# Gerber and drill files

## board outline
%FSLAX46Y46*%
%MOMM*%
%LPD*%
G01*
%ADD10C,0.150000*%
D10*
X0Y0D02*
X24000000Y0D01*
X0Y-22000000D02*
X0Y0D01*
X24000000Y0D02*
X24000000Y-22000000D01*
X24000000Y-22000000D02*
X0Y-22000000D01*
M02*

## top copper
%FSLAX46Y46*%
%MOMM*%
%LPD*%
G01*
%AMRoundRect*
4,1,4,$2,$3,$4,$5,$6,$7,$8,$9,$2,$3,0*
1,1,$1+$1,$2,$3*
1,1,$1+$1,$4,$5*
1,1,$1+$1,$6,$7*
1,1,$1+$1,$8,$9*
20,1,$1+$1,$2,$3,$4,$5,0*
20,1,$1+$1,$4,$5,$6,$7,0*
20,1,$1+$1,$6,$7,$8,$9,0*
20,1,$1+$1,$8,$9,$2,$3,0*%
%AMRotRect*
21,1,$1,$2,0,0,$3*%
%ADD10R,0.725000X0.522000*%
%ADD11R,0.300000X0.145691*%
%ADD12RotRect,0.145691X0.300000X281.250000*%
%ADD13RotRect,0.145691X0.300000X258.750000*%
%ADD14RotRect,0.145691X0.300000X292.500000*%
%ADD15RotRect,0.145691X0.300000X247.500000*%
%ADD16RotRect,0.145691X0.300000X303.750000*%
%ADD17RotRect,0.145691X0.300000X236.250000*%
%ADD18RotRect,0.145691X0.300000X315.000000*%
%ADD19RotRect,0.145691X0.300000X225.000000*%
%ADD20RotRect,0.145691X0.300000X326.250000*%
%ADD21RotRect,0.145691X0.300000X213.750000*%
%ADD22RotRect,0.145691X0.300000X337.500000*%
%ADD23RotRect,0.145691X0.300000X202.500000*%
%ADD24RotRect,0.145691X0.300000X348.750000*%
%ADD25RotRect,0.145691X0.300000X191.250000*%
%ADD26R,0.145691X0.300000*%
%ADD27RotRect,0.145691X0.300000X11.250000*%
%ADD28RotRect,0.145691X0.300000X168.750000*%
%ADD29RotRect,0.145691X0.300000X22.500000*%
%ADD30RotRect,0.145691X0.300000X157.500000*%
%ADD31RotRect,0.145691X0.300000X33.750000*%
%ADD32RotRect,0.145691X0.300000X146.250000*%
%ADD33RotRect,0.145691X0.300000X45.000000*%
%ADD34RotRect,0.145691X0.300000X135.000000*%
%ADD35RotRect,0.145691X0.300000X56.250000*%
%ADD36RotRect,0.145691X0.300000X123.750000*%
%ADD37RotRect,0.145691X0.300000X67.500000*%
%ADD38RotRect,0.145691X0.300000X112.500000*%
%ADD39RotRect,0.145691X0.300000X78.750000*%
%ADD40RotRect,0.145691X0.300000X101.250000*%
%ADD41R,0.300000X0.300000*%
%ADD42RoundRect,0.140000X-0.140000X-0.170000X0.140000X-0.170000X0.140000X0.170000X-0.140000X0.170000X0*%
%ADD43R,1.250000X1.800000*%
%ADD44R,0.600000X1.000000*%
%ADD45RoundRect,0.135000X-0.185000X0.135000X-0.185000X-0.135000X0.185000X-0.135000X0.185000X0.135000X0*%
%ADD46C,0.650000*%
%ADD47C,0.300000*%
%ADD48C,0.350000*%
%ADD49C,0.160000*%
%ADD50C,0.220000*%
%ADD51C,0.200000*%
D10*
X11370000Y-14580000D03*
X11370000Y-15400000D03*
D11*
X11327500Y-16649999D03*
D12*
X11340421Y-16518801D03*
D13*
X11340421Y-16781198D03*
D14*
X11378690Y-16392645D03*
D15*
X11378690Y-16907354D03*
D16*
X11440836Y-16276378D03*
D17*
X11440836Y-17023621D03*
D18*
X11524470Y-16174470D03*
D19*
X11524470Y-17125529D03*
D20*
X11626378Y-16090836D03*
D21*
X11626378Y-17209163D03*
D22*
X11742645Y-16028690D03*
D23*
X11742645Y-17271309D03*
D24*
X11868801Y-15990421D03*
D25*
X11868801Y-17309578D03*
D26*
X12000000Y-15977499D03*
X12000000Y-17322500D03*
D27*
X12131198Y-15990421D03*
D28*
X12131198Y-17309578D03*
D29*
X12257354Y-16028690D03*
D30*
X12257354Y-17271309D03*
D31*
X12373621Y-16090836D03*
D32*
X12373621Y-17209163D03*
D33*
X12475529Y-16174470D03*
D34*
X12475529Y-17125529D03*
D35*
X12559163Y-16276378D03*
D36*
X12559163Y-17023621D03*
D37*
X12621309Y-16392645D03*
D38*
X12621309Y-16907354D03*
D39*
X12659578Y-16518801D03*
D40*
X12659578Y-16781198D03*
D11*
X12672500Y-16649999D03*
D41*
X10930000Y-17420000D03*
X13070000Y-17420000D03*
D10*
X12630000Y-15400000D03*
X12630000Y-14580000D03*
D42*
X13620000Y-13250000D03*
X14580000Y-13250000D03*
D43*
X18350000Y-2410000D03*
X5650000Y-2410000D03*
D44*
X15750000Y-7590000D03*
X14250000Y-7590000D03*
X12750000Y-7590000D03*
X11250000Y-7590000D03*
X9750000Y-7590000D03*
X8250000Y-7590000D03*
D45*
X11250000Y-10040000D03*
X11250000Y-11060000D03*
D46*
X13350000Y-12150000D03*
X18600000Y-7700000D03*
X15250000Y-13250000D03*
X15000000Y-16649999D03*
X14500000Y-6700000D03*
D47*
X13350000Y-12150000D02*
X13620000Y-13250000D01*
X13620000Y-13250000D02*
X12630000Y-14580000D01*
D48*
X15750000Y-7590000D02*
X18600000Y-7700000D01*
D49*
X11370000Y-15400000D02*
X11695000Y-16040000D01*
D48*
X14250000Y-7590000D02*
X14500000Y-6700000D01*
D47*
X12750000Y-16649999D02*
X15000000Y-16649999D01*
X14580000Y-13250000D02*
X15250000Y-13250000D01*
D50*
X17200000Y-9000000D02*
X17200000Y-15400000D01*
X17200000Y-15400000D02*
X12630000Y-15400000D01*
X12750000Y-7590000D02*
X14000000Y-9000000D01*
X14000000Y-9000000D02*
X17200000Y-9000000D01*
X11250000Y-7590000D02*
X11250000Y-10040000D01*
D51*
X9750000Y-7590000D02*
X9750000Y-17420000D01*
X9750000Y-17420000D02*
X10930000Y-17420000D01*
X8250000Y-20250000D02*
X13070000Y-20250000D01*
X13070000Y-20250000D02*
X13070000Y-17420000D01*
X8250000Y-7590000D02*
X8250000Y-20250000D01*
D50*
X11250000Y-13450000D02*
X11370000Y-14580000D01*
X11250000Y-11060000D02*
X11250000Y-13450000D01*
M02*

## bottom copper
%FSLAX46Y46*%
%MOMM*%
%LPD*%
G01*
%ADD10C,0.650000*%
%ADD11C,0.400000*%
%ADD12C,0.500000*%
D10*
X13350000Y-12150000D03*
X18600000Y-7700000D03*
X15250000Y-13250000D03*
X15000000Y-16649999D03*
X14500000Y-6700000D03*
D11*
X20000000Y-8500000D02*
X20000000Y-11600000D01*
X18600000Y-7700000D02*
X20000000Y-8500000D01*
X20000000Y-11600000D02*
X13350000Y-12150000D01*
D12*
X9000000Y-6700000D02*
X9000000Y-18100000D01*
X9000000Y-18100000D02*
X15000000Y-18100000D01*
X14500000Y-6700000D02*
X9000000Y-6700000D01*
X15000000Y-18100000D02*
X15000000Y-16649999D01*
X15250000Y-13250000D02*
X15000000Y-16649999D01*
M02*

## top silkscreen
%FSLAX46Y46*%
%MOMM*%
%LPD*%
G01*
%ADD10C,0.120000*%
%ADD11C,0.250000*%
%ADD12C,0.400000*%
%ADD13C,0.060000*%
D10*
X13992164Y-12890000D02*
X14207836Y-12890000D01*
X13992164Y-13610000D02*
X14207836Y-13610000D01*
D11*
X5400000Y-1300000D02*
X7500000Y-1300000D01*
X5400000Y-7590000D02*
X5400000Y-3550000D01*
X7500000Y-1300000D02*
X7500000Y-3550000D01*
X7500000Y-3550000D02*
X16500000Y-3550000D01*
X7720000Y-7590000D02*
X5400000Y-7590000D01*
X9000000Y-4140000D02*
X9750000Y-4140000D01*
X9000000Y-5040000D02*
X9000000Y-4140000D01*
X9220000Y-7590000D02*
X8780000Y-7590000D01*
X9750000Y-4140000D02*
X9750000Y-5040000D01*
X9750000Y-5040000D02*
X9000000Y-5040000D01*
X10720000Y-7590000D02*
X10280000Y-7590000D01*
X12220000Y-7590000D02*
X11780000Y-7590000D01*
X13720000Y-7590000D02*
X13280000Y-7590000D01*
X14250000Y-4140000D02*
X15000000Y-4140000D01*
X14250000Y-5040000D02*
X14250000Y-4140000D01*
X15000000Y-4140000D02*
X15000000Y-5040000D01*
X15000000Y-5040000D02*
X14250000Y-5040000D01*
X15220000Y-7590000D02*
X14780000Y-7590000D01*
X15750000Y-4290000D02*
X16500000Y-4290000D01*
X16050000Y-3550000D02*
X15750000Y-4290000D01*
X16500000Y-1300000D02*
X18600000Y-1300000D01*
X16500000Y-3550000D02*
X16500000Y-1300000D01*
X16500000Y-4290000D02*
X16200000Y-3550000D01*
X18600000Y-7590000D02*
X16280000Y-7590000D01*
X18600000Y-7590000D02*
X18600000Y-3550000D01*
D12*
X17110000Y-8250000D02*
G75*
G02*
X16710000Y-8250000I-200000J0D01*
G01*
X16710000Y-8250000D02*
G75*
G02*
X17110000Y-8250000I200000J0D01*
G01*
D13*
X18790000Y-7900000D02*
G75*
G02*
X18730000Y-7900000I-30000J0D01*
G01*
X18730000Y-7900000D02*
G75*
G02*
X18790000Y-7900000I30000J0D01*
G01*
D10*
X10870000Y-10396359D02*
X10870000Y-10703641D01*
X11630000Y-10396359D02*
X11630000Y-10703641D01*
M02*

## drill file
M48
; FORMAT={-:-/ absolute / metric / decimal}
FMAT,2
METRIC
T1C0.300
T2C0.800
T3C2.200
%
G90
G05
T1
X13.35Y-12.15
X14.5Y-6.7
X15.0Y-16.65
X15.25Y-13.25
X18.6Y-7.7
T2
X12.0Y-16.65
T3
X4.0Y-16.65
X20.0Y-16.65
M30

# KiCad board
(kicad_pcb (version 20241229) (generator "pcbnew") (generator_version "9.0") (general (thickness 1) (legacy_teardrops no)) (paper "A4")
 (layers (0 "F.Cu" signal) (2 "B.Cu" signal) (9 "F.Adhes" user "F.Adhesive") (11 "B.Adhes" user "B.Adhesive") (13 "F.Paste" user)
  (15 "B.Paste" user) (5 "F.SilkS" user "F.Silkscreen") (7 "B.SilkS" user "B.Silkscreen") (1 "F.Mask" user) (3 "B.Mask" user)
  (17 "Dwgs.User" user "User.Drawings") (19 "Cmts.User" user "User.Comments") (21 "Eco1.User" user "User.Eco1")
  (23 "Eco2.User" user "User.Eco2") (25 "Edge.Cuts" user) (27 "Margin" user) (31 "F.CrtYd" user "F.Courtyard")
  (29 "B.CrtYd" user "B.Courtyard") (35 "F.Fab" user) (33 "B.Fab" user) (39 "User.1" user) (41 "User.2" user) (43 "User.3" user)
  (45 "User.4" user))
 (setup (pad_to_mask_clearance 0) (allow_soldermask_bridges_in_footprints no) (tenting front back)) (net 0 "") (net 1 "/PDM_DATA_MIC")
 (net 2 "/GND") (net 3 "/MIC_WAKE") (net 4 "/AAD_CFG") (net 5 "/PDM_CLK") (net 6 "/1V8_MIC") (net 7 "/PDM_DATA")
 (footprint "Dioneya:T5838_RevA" (layer "F.Cu") (at 12 16)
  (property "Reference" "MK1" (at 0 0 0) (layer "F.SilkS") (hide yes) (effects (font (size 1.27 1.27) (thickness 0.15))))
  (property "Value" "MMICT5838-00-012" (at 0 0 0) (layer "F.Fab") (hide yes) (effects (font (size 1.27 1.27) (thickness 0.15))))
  (pad "" np_thru_hole circle (at 0 0.649999) (size 0.8 0.8) (drill 0.8) (layers "*.Cu" "*.Mask"))
  (pad "1" smd rect (at -0.63 -1.42 90) (size 0.522 0.725) (layers "F.Cu" "F.Mask" "F.Paste") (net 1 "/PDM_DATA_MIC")
   (solder_paste_margin -0.05) (thermal_bridge_angle 45))
  (pad "2" smd rect (at -0.63 -0.6 90) (size 0.522 0.725) (layers "F.Cu" "F.Mask" "F.Paste") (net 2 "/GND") (solder_paste_margin -0.05)
   (thermal_bridge_angle 45))
  (pad "3" smd rect (at -0.6725 0.649999 270) (size 0.145691 0.3) (layers "F.Cu" "F.Mask") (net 2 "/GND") (thermal_bridge_angle 45))
  (pad "3" smd rect (at -0.659579 0.518801 281.25) (size 0.145691 0.3) (layers "F.Cu" "F.Mask") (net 2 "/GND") (thermal_bridge_angle 45))
  (pad "3" smd rect (at -0.659579 0.781198 258.75) (size 0.145691 0.3) (layers "F.Cu" "F.Mask") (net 2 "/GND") (thermal_bridge_angle 45))
  (pad "3" smd rect (at -0.62131 0.392645 292.5) (size 0.145691 0.3) (layers "F.Cu" "F.Mask") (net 2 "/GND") (thermal_bridge_angle 45))
  (pad "3" smd rect (at -0.62131 0.907354 247.5) (size 0.145691 0.3) (layers "F.Cu" "F.Mask") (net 2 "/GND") (thermal_bridge_angle 45))
  (pad "3" smd rect (at -0.559164 0.276378 303.75) (size 0.145691 0.3) (layers "F.Cu" "F.Mask") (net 2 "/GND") (thermal_bridge_angle 45))
  (pad "3" smd rect (at -0.559164 1.023621 236.25) (size 0.145691 0.3) (layers "F.Cu" "F.Mask") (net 2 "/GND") (thermal_bridge_angle 45))
  (pad "3" smd rect (at -0.47553 0.17447 315) (size 0.145691 0.3) (layers "F.Cu" "F.Mask") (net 2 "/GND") (thermal_bridge_angle 45))
  (pad "3" smd rect (at -0.47553 1.125529 225) (size 0.145691 0.3) (layers "F.Cu" "F.Mask") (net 2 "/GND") (thermal_bridge_angle 45))
  (pad "3" smd rect (at -0.373622 0.090836 326.25) (size 0.145691 0.3) (layers "F.Cu" "F.Mask") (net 2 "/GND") (thermal_bridge_angle 45))
  (pad "3" smd rect (at -0.373622 1.209163 213.75) (size 0.145691 0.3) (layers "F.Cu" "F.Mask") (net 2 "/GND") (thermal_bridge_angle 45))
  (pad "3" smd rect (at -0.257355 0.02869 337.5) (size 0.145691 0.3) (layers "F.Cu" "F.Mask") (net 2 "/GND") (thermal_bridge_angle 45))
  (pad "3" smd rect (at -0.257355 1.271309 202.5) (size 0.145691 0.3) (layers "F.Cu" "F.Mask") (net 2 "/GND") (thermal_bridge_angle 45))
  (pad "3" smd rect (at -0.131199 -0.009579 348.75) (size 0.145691 0.3) (layers "F.Cu" "F.Mask") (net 2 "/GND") (thermal_bridge_angle 45))
  (pad "3" smd rect (at -0.131199 1.309578 191.25) (size 0.145691 0.3) (layers "F.Cu" "F.Mask") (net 2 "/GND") (thermal_bridge_angle 45))
  (pad "3" smd rect (at 0 -0.022501) (size 0.145691 0.3) (layers "F.Cu" "F.Mask") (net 2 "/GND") (thermal_bridge_angle 45))
  (pad "3" smd rect (at 0 1.3225 180) (size 0.145691 0.3) (layers "F.Cu" "F.Mask") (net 2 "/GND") (thermal_bridge_angle 45))
  (pad "3" smd rect (at 0.131198 -0.009579 11.25) (size 0.145691 0.3) (layers "F.Cu" "F.Mask") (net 2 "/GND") (thermal_bridge_angle 45))
  (pad "3" smd rect (at 0.131198 1.309578 168.75) (size 0.145691 0.3) (layers "F.Cu" "F.Mask") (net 2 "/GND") (thermal_bridge_angle 45))
  (pad "3" smd rect (at 0.257354 0.02869 22.5) (size 0.145691 0.3) (layers "F.Cu" "F.Mask") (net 2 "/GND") (thermal_bridge_angle 45))
  (pad "3" smd rect (at 0.257354 1.271309 157.5) (size 0.145691 0.3) (layers "F.Cu" "F.Mask") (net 2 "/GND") (thermal_bridge_angle 45))
  (pad "3" smd rect (at 0.373621 0.090836 33.75) (size 0.145691 0.3) (layers "F.Cu" "F.Mask") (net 2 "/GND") (thermal_bridge_angle 45))
  (pad "3" smd rect (at 0.373621 1.209163 146.25) (size 0.145691 0.3) (layers "F.Cu" "F.Mask") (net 2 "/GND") (thermal_bridge_angle 45))
  (pad "3" smd rect (at 0.475529 0.17447 45) (size 0.145691 0.3) (layers "F.Cu" "F.Mask") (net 2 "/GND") (thermal_bridge_angle 45))
  (pad "3" smd rect (at 0.475529 1.125529 135) (size 0.145691 0.3) (layers "F.Cu" "F.Mask") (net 2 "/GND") (thermal_bridge_angle 45))
  (pad "3" smd rect (at 0.559163 0.276378 56.25) (size 0.145691 0.3) (layers "F.Cu" "F.Mask") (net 2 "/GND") (thermal_bridge_angle 45))
  (pad "3" smd rect (at 0.559163 1.023621 123.75) (size 0.145691 0.3) (layers "F.Cu" "F.Mask") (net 2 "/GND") (thermal_bridge_angle 45))
  (pad "3" smd rect (at 0.621309 0.392645 67.5) (size 0.145691 0.3) (layers "F.Cu" "F.Mask") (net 2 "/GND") (thermal_bridge_angle 45))
  (pad "3" smd rect (at 0.621309 0.907354 112.5) (size 0.145691 0.3) (layers "F.Cu" "F.Mask") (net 2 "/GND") (thermal_bridge_angle 45))
  (pad "3" smd rect (at 0.659578 0.518801 78.75) (size 0.145691 0.3) (layers "F.Cu" "F.Mask") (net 2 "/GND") (thermal_bridge_angle 45))
  (pad "3" smd rect (at 0.659578 0.781198 101.25) (size 0.145691 0.3) (layers "F.Cu" "F.Mask") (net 2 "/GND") (thermal_bridge_angle 45))
  (pad "3" smd rect (at 0.6725 0.649999 90) (size 0.145691 0.3) (layers "F.Cu" "F.Mask") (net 2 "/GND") (thermal_bridge_angle 45))
  (pad "4" smd rect (at -1.07 1.42 90) (size 0.3 0.3) (layers "F.Cu" "F.Mask" "F.Paste") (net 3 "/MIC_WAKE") (solder_paste_margin -0.015)
   (thermal_bridge_angle 45))
  (pad "5" smd rect (at 1.07 1.42 90) (size 0.3 0.3) (layers "F.Cu" "F.Mask" "F.Paste") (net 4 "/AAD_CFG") (solder_paste_margin -0.015)
   (thermal_bridge_angle 45))
  (pad "6" smd rect (at 0.63 -0.6 90) (size 0.522 0.725) (layers "F.Cu" "F.Mask" "F.Paste") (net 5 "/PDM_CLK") (solder_paste_margin -0.05)
   (thermal_bridge_angle 45))
  (pad "7" smd rect (at 0.63 -1.42 90) (size 0.522 0.725) (layers "F.Cu" "F.Mask" "F.Paste") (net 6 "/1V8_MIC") (solder_paste_margin -0.05)
   (thermal_bridge_angle 45)))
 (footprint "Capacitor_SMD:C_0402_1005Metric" (layer "F.Cu") (at 14.1 13.25)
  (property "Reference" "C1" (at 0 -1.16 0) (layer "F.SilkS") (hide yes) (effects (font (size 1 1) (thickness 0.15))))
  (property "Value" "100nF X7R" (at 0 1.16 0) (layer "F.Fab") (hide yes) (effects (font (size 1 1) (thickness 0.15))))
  (fp_line (start -0.107836 -0.36) (end 0.107836 -0.36) (stroke (width 0.12) (type solid)) (layer "F.SilkS"))
  (fp_line (start -0.107836 0.36) (end 0.107836 0.36) (stroke (width 0.12) (type solid)) (layer "F.SilkS"))
  (pad "1" smd roundrect (at -0.48 0) (size 0.56 0.62) (layers "F.Cu" "F.Mask" "F.Paste") (roundrect_rratio 0.25) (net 6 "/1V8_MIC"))
  (pad "2" smd roundrect (at 0.48 0) (size 0.56 0.62) (layers "F.Cu" "F.Mask" "F.Paste") (roundrect_rratio 0.25) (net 2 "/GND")))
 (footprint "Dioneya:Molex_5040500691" (layer "F.Cu") (at 12 5 180)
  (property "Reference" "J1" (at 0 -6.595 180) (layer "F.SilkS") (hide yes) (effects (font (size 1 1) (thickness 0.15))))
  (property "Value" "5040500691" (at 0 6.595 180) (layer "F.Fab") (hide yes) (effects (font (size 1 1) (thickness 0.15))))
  (fp_line (start 6.6 3.7) (end 4.5 3.7) (stroke (width 0.25) (type solid)) (layer "F.SilkS"))
  (fp_line (start 6.6 -2.59) (end 6.6 1.45) (stroke (width 0.25) (type solid)) (layer "F.SilkS"))
  (fp_line (start 4.5 3.7) (end 4.5 1.45) (stroke (width 0.25) (type solid)) (layer "F.SilkS"))
  (fp_line (start 4.5 1.45) (end -4.5 1.45) (stroke (width 0.25) (type solid)) (layer "F.SilkS"))
  (fp_line (start 4.28 -2.59) (end 6.6 -2.59) (stroke (width 0.25) (type solid)) (layer "F.SilkS"))
  (fp_line (start 3 0.86) (end 2.25 0.86) (stroke (width 0.25) (type solid)) (layer "F.SilkS"))
  (fp_line (start 3 -0.04) (end 3 0.86) (stroke (width 0.25) (type solid)) (layer "F.SilkS"))
  (fp_line (start 2.78 -2.59) (end 3.22 -2.59) (stroke (width 0.25) (type solid)) (layer "F.SilkS"))
  (fp_line (start 2.25 0.86) (end 2.25 -0.04) (stroke (width 0.25) (type solid)) (layer "F.SilkS"))
  (fp_line (start 2.25 -0.04) (end 3 -0.04) (stroke (width 0.25) (type solid)) (layer "F.SilkS"))
  (fp_line (start 1.28 -2.59) (end 1.72 -2.59) (stroke (width 0.25) (type solid)) (layer "F.SilkS"))
  (fp_line (start -0.22 -2.59) (end 0.22 -2.59) (stroke (width 0.25) (type solid)) (layer "F.SilkS"))
  (fp_line (start -1.72 -2.59) (end -1.28 -2.59) (stroke (width 0.25) (type solid)) (layer "F.SilkS"))
  (fp_line (start -2.25 0.86) (end -3 0.86) (stroke (width 0.25) (type solid)) (layer "F.SilkS"))
  (fp_line (start -2.25 -0.04) (end -2.25 0.86) (stroke (width 0.25) (type solid)) (layer "F.SilkS"))
  (fp_line (start -3 0.86) (end -3 -0.04) (stroke (width 0.25) (type solid)) (layer "F.SilkS"))
  (fp_line (start -3 -0.04) (end -2.25 -0.04) (stroke (width 0.25) (type solid)) (layer "F.SilkS"))
  (fp_line (start -3.22 -2.59) (end -2.78 -2.59) (stroke (width 0.25) (type solid)) (layer "F.SilkS"))
  (fp_line (start -3.75 0.71) (end -4.5 0.71) (stroke (width 0.25) (type solid)) (layer "F.SilkS"))
  (fp_line (start -4.05 1.45) (end -3.75 0.71) (stroke (width 0.25) (type solid)) (layer "F.SilkS"))
  (fp_line (start -4.5 3.7) (end -6.6 3.7) (stroke (width 0.25) (type solid)) (layer "F.SilkS"))
  (fp_line (start -4.5 1.45) (end -4.5 3.7) (stroke (width 0.25) (type solid)) (layer "F.SilkS"))
  (fp_line (start -4.5 0.71) (end -4.2 1.45) (stroke (width 0.25) (type solid)) (layer "F.SilkS"))
  (fp_line (start -6.6 -2.59) (end -4.28 -2.59) (stroke (width 0.25) (type solid)) (layer "F.SilkS"))
  (fp_line (start -6.6 -2.59) (end -6.6 1.45) (stroke (width 0.25) (type solid)) (layer "F.SilkS"))
  (fp_circle (center -4.91 -3.25) (end -4.71 -3.25) (stroke (width 0.4) (type solid)) (fill no) (layer "F.SilkS"))
  (fp_circle (center -6.76 -2.9) (end -6.73 -2.9) (stroke (width 0.06) (type solid)) (fill no) (layer "F.SilkS"))
  (pad "" smd rect (at -6.35 2.59) (size 1.25 1.8) (layers "F.Cu" "F.Mask" "F.Paste"))
  (pad "" smd rect (at 6.35 2.59) (size 1.25 1.8) (layers "F.Cu" "F.Mask" "F.Paste"))
  (pad "1" smd rect (at -3.75 -2.59) (size 0.6 1) (layers "F.Cu" "F.Mask" "F.Paste") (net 6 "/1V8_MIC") (solder_paste_margin 0))
  (pad "2" smd rect (at -2.25 -2.59) (size 0.6 1) (layers "F.Cu" "F.Mask" "F.Paste") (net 2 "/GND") (solder_paste_margin 0))
  (pad "3" smd rect (at -0.75 -2.59) (size 0.6 1) (layers "F.Cu" "F.Mask" "F.Paste") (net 5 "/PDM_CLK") (solder_paste_margin 0))
  (pad "4" smd rect (at 0.75 -2.59) (size 0.6 1) (layers "F.Cu" "F.Mask" "F.Paste") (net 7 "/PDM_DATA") (solder_paste_margin 0))
  (pad "5" smd rect (at 2.25 -2.59) (size 0.6 1) (layers "F.Cu" "F.Mask" "F.Paste") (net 3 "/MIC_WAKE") (solder_paste_margin 0))
  (pad "6" smd rect (at 3.75 -2.59) (size 0.6 1) (layers "F.Cu" "F.Mask" "F.Paste") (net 4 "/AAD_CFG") (solder_paste_margin 0)))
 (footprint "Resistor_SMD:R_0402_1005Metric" (layer "F.Cu") (at 11.25 10.55 -90)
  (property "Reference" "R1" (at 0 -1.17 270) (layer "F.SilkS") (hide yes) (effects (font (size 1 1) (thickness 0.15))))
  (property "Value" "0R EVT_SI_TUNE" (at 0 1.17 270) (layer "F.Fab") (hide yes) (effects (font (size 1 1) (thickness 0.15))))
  (fp_line (start -0.153641 0.38) (end 0.153641 0.38) (stroke (width 0.12) (type solid)) (layer "F.SilkS"))
  (fp_line (start -0.153641 -0.38) (end 0.153641 -0.38) (stroke (width 0.12) (type solid)) (layer "F.SilkS"))
  (pad "1" smd roundrect (at -0.51 0 270) (size 0.54 0.64) (layers "F.Cu" "F.Mask" "F.Paste") (roundrect_rratio 0.25) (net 7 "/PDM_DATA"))
  (pad "2" smd roundrect (at 0.51 0 270) (size 0.54 0.64) (layers "F.Cu" "F.Mask" "F.Paste") (roundrect_rratio 0.25) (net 1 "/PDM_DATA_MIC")))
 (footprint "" (layer "F.Cu") (at 4 16.649999)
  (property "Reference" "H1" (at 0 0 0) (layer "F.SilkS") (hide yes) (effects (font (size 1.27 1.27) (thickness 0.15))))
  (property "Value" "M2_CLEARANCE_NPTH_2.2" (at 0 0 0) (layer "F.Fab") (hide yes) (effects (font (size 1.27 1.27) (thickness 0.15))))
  (pad "" np_thru_hole circle (at 0 0) (size 2.2 2.2) (drill 2.2) (layers "*.Cu" "*.Mask")))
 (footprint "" (layer "F.Cu") (at 20 16.649999)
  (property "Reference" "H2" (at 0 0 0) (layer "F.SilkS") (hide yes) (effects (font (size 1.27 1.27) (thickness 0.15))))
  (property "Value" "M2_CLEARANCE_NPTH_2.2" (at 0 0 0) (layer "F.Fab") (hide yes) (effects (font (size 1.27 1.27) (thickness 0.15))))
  (pad "" np_thru_hole circle (at 0 0) (size 2.2 2.2) (drill 2.2) (layers "*.Cu" "*.Mask")))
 (gr_line (start 0 0) (end 24 0) (stroke (width 0.15) (type default)) (layer "Edge.Cuts"))
 (gr_line (start 0 22) (end 0 0) (stroke (width 0.15) (type default)) (layer "Edge.Cuts"))
 (gr_line (start 24 0) (end 24 22) (stroke (width 0.15) (type default)) (layer "Edge.Cuts"))
 (gr_line (start 24 22) (end 0 22) (stroke (width 0.15) (type default)) (layer "Edge.Cuts"))
 (segment (start 13.35 12.15) (end 13.62 13.25) (width 0.3) (layer "F.Cu") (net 6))
 (segment (start 13.62 13.25) (end 12.63 14.58) (width 0.3) (layer "F.Cu") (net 6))
 (segment (start 15.75 7.59) (end 18.6 7.7) (width 0.35) (layer "F.Cu") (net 6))
 (via (at 13.35 12.15) (size 0.65) (drill 0.3) (layers "F.Cu" "B.Cu") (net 6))
 (via (at 18.6 7.7) (size 0.65) (drill 0.3) (layers "F.Cu" "B.Cu") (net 6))
 (segment (start 20 8.5) (end 20 11.6) (width 0.4) (layer "B.Cu") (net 6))
 (segment (start 18.6 7.7) (end 20 8.5) (width 0.4) (layer "B.Cu") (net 6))
 (segment (start 20 11.6) (end 13.35 12.15) (width 0.4) (layer "B.Cu") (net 6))
 (segment (start 11.37 15.4) (end 11.695 16.04) (width 0.16) (layer "F.Cu") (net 2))
 (segment (start 14.25 7.59) (end 14.5 6.7) (width 0.35) (layer "F.Cu") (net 2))
 (segment (start 12.75 16.649999) (end 15 16.649999) (width 0.3) (layer "F.Cu") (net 2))
 (segment (start 14.58 13.25) (end 15.25 13.25) (width 0.3) (layer "F.Cu") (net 2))
 (via (at 15.25 13.25) (size 0.65) (drill 0.3) (layers "F.Cu" "B.Cu") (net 2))
 (via (at 15 16.649999) (size 0.65) (drill 0.3) (layers "F.Cu" "B.Cu") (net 2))
 (via (at 14.5 6.7) (size 0.65) (drill 0.3) (layers "F.Cu" "B.Cu") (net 2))
 (segment (start 9 6.7) (end 9 18.1) (width 0.5) (layer "B.Cu") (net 2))
 (segment (start 9 18.1) (end 15 18.1) (width 0.5) (layer "B.Cu") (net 2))
 (segment (start 14.5 6.7) (end 9 6.7) (width 0.5) (layer "B.Cu") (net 2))
 (segment (start 15 18.1) (end 15 16.649999) (width 0.5) (layer "B.Cu") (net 2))
 (segment (start 15.25 13.25) (end 15 16.649999) (width 0.5) (layer "B.Cu") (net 2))
 (segment (start 17.2 9) (end 17.2 15.4) (width 0.22) (layer "F.Cu") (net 5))
 (segment (start 17.2 15.4) (end 12.63 15.4) (width 0.22) (layer "F.Cu") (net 5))
 (segment (start 12.75 7.59) (end 14 9) (width 0.22) (layer "F.Cu") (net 5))
 (segment (start 14 9) (end 17.2 9) (width 0.22) (layer "F.Cu") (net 5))
 (segment (start 11.25 7.59) (end 11.25 10.04) (width 0.22) (layer "F.Cu") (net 7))
 (segment (start 9.75 7.59) (end 9.75 17.42) (width 0.2) (layer "F.Cu") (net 3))
 (segment (start 9.75 17.42) (end 10.93 17.42) (width 0.2) (layer "F.Cu") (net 3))
 (segment (start 8.25 20.25) (end 13.07 20.25) (width 0.2) (layer "F.Cu") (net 4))
 (segment (start 13.07 20.25) (end 13.07 17.42) (width 0.2) (layer "F.Cu") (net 4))
 (segment (start 8.25 7.59) (end 8.25 20.25) (width 0.2) (layer "F.Cu") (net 4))
 (segment (start 11.25 13.45) (end 11.37 14.58) (width 0.22) (layer "F.Cu") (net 1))
 (segment (start 11.25 11.06) (end 11.25 13.45) (width 0.22) (layer "F.Cu") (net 1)))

